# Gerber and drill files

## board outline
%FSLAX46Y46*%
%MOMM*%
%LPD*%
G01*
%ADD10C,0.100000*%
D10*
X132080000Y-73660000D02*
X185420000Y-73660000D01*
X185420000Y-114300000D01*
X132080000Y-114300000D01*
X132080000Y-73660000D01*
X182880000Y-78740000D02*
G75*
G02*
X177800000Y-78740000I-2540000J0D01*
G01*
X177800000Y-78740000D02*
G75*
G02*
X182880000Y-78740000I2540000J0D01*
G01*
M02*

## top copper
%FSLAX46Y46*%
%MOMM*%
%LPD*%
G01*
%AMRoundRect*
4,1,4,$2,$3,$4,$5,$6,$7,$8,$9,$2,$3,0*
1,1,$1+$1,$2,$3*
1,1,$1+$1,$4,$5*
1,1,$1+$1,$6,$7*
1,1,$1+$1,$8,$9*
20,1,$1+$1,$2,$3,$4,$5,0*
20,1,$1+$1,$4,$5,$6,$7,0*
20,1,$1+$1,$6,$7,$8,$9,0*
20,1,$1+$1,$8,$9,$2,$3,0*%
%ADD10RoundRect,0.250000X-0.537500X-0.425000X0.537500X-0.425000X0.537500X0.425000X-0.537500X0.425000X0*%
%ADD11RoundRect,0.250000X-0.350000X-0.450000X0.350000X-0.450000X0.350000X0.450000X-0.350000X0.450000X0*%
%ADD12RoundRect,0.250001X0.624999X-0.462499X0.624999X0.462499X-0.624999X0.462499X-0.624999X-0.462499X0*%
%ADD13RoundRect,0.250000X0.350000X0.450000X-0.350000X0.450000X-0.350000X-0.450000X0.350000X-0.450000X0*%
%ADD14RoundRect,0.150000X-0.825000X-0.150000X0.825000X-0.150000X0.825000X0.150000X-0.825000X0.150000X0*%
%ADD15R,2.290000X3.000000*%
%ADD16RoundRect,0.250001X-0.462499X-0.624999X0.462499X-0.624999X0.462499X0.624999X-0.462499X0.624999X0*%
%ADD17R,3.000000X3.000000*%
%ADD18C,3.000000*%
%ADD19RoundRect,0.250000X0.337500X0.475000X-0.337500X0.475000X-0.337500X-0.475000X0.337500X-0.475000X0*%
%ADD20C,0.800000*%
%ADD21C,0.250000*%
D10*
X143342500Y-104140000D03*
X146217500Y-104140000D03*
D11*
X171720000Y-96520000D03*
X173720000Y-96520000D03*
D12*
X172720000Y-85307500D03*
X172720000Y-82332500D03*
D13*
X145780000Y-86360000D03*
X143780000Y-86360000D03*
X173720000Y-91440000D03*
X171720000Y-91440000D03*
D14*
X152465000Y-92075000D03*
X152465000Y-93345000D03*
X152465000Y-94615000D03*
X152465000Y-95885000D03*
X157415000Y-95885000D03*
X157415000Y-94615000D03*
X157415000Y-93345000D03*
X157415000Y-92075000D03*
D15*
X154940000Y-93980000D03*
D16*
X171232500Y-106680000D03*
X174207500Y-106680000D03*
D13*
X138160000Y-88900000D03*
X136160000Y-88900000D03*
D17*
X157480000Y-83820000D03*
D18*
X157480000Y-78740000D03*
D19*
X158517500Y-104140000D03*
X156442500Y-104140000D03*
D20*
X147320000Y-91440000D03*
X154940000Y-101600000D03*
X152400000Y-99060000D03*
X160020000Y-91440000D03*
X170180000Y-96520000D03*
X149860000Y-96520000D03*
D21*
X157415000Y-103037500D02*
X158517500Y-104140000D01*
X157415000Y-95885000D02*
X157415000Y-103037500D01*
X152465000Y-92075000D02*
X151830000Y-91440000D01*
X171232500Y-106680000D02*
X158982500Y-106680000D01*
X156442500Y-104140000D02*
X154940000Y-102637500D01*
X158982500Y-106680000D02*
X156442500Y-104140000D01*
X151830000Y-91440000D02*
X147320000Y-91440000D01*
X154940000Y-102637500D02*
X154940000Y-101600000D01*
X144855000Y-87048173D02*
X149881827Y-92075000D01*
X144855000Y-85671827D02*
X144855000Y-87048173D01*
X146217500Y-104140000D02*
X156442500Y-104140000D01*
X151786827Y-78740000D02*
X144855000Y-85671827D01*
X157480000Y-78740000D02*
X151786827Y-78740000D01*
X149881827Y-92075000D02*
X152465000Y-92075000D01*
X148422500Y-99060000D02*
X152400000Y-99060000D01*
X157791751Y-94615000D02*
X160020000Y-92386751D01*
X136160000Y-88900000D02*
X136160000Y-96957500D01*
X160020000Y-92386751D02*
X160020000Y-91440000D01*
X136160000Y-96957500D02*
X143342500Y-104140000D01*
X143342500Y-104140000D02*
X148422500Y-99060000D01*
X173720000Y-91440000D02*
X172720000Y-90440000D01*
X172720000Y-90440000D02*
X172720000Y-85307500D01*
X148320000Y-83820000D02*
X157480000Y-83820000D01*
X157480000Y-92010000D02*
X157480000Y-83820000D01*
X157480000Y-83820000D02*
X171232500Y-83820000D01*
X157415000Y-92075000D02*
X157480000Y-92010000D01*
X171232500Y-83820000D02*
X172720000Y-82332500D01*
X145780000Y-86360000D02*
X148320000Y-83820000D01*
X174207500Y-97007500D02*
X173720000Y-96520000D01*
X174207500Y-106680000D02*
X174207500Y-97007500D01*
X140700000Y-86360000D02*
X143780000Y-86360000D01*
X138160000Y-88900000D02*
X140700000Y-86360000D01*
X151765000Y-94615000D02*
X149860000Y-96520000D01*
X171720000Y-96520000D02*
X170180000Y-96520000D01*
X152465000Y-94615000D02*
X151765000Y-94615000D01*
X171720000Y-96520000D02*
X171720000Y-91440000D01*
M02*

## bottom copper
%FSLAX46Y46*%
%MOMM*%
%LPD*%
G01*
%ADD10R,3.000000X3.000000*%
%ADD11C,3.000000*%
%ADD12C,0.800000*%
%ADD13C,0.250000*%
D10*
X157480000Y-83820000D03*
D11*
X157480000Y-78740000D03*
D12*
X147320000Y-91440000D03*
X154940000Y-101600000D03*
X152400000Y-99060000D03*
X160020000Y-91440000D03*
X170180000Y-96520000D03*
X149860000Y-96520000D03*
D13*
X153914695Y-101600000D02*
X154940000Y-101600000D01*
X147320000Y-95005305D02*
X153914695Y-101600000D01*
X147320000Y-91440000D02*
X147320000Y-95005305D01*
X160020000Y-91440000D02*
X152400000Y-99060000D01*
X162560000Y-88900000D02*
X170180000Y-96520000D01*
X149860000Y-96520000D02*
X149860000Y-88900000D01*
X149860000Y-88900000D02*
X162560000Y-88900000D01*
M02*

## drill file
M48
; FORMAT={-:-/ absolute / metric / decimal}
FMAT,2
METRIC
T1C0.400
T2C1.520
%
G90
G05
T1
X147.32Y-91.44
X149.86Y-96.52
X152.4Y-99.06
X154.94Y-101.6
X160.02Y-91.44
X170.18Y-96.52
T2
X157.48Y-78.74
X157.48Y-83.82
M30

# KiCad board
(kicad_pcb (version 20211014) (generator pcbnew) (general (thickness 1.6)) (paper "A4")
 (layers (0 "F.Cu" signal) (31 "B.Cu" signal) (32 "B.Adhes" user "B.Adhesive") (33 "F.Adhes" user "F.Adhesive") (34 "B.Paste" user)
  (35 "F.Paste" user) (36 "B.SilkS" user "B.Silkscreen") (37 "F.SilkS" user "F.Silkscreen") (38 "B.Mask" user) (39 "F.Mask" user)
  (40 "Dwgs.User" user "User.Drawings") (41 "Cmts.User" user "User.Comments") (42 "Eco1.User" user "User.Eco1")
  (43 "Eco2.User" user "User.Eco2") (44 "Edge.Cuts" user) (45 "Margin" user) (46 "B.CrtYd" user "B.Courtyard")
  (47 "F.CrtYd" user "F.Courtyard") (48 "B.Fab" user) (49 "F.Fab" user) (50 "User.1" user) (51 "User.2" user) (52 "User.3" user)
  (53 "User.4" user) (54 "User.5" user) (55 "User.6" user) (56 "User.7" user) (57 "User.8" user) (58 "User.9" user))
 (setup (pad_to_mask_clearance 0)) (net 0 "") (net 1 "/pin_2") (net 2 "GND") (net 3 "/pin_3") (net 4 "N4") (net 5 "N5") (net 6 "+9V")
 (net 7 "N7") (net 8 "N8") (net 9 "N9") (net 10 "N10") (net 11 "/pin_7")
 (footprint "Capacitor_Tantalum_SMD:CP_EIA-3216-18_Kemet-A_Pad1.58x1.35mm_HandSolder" (layer "F.Cu") (at 144.78 104.14)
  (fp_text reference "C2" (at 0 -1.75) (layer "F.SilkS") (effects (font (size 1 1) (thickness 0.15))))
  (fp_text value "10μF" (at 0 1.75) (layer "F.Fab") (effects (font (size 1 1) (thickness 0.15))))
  (pad "1" smd roundrect (at -1.4375 0) (size 1.575 1.35) (layers "F.Cu" "F.Paste" "F.Mask") (roundrect_rratio 0.185185) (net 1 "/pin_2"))
  (pad "2" smd roundrect (at 1.4375 0) (size 1.575 1.35) (layers "F.Cu" "F.Paste" "F.Mask") (roundrect_rratio 0.185185) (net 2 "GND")))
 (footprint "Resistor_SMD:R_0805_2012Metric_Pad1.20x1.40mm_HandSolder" (layer "F.Cu") (at 172.72 96.52)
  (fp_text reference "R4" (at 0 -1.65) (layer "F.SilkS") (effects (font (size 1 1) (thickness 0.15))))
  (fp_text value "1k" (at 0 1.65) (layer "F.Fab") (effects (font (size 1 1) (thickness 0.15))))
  (pad "1" smd roundrect (at -1 0) (size 1.2 1.4) (layers "F.Cu" "F.Paste" "F.Mask") (roundrect_rratio 0.208333) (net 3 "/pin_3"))
  (pad "2" smd roundrect (at 1 0) (size 1.2 1.4) (layers "F.Cu" "F.Paste" "F.Mask") (roundrect_rratio 0.208333) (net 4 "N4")))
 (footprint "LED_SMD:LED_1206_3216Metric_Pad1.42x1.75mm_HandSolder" (layer "F.Cu") (at 172.72 83.82 90)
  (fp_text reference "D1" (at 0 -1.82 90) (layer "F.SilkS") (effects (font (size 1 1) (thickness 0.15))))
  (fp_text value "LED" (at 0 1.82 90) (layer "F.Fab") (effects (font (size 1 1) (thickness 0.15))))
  (pad "1" smd roundrect (at -1.4875 0 90) (size 1.425 1.75) (layers "F.Cu" "F.Paste" "F.Mask") (roundrect_rratio 0.175439) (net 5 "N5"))
  (pad "2" smd roundrect (at 1.4875 0 90) (size 1.425 1.75) (layers "F.Cu" "F.Paste" "F.Mask") (roundrect_rratio 0.175439) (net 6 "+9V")))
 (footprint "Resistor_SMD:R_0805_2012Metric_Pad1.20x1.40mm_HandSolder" (layer "F.Cu") (at 144.78 86.36 180)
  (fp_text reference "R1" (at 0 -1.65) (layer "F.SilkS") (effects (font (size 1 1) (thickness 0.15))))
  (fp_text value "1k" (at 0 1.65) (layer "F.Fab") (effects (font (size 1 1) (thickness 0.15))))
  (pad "1" smd roundrect (at -1 0 180) (size 1.2 1.4) (layers "F.Cu" "F.Paste" "F.Mask") (roundrect_rratio 0.208333) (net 6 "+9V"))
  (pad "2" smd roundrect (at 1 0 180) (size 1.2 1.4) (layers "F.Cu" "F.Paste" "F.Mask") (roundrect_rratio 0.208333) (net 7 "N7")))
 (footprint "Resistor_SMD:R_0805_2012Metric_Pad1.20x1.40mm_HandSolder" (layer "F.Cu") (at 172.72 91.44 180)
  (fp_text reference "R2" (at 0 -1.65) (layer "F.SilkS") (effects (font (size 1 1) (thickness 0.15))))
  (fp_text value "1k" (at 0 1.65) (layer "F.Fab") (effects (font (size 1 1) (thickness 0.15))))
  (pad "1" smd roundrect (at -1 0 180) (size 1.2 1.4) (layers "F.Cu" "F.Paste" "F.Mask") (roundrect_rratio 0.208333) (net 5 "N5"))
  (pad "2" smd roundrect (at 1 0 180) (size 1.2 1.4) (layers "F.Cu" "F.Paste" "F.Mask") (roundrect_rratio 0.208333) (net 3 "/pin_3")))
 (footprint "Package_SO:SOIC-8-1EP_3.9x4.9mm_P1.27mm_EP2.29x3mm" (layer "F.Cu") (at 154.94 93.98)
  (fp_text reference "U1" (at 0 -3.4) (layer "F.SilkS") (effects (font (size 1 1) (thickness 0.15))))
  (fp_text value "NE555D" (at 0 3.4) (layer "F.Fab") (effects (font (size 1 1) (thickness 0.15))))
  (pad "" smd roundrect (at 0.57 -0.75) (size 0.92 1.21) (layers "F.Paste") (roundrect_rratio 0.25))
  (pad "" smd roundrect (at 0.57 0.75) (size 0.92 1.21) (layers "F.Paste") (roundrect_rratio 0.25))
  (pad "" smd roundrect (at -0.57 0.75) (size 0.92 1.21) (layers "F.Paste") (roundrect_rratio 0.25))
  (pad "" smd roundrect (at -0.57 -0.75) (size 0.92 1.21) (layers "F.Paste") (roundrect_rratio 0.25))
  (pad "1" smd roundrect (at -2.475 -1.905) (size 1.95 0.6) (layers "F.Cu" "F.Paste" "F.Mask") (roundrect_rratio 0.25) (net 2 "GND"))
  (pad "2" smd roundrect (at -2.475 -0.635) (size 1.95 0.6) (layers "F.Cu" "F.Paste" "F.Mask") (roundrect_rratio 0.25) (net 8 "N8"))
  (pad "3" smd roundrect (at -2.475 0.635) (size 1.95 0.6) (layers "F.Cu" "F.Paste" "F.Mask") (roundrect_rratio 0.25) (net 3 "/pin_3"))
  (pad "4" smd roundrect (at -2.475 1.905) (size 1.95 0.6) (layers "F.Cu" "F.Paste" "F.Mask") (roundrect_rratio 0.25) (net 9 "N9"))
  (pad "5" smd roundrect (at 2.475 1.905) (size 1.95 0.6) (layers "F.Cu" "F.Paste" "F.Mask") (roundrect_rratio 0.25) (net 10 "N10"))
  (pad "6" smd roundrect (at 2.475 0.635) (size 1.95 0.6) (layers "F.Cu" "F.Paste" "F.Mask") (roundrect_rratio 0.25) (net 1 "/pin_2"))
  (pad "7" smd roundrect (at 2.475 -0.635) (size 1.95 0.6) (layers "F.Cu" "F.Paste" "F.Mask") (roundrect_rratio 0.25) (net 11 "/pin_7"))
  (pad "8" smd roundrect (at 2.475 -1.905) (size 1.95 0.6) (layers "F.Cu" "F.Paste" "F.Mask") (roundrect_rratio 0.25) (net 6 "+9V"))
  (pad "9" smd rect (at 0 0) (size 2.29 3) (layers "F.Cu" "F.Mask")))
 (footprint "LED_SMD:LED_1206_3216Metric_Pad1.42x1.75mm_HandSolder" (layer "F.Cu") (at 172.72 106.68)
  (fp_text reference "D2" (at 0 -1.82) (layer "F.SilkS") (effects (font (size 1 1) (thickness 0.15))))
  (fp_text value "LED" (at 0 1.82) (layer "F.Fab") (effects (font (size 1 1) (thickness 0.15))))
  (pad "1" smd roundrect (at -1.4875 0) (size 1.425 1.75) (layers "F.Cu" "F.Paste" "F.Mask") (roundrect_rratio 0.175439) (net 2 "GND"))
  (pad "2" smd roundrect (at 1.4875 0) (size 1.425 1.75) (layers "F.Cu" "F.Paste" "F.Mask") (roundrect_rratio 0.175439) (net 4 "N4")))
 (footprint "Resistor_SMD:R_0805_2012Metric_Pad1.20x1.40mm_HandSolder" (layer "F.Cu") (at 137.16 88.9 180)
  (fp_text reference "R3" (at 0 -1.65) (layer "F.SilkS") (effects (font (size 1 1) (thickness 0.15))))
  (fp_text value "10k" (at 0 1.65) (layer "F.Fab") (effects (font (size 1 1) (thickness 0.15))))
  (pad "1" smd roundrect (at -1 0 180) (size 1.2 1.4) (layers "F.Cu" "F.Paste" "F.Mask") (roundrect_rratio 0.208333) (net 7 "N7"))
  (pad "2" smd roundrect (at 1 0 180) (size 1.2 1.4) (layers "F.Cu" "F.Paste" "F.Mask") (roundrect_rratio 0.208333) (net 1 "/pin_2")))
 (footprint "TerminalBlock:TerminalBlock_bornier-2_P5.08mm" (layer "F.Cu") (at 157.48 83.82 90)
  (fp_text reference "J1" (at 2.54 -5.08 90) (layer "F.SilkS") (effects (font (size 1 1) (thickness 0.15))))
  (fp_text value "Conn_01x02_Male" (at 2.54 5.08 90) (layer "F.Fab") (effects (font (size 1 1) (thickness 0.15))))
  (pad "1" thru_hole rect (at 0 0 90) (size 3 3) (drill 1.52) (layers *.Cu *.Mask) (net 6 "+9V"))
  (pad "2" thru_hole circle (at 5.08 0 90) (size 3 3) (drill 1.52) (layers *.Cu *.Mask) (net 2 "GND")))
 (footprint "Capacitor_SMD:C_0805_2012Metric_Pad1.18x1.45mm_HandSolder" (layer "F.Cu") (at 157.48 104.14 180)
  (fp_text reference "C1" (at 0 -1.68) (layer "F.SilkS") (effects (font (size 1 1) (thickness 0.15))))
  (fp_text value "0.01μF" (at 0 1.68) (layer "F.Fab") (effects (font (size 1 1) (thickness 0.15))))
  (pad "1" smd roundrect (at -1.0375 0 180) (size 1.175 1.45) (layers "F.Cu" "F.Paste" "F.Mask") (roundrect_rratio 0.212766) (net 10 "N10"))
  (pad "2" smd roundrect (at 1.0375 0 180) (size 1.175 1.45) (layers "F.Cu" "F.Paste" "F.Mask") (roundrect_rratio 0.212766) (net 2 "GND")))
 (gr_rect (start 185.42 114.3) (end 132.08 73.66) (layer "Edge.Cuts") (width 0.1) (fill none))
 (gr_circle (center 180.34 78.74) (end 180.34 81.28) (layer "Edge.Cuts") (width 0.1) (fill none))
 (segment (start 157.415 103.0375) (end 158.5175 104.14) (width 0.25) (layer "F.Cu") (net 10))
 (segment (start 157.415 95.885) (end 157.415 103.0375) (width 0.25) (layer "F.Cu") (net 10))
 (segment (start 152.465 92.075) (end 151.83 91.44) (width 0.25) (layer "F.Cu") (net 2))
 (segment (start 171.2325 106.68) (end 158.9825 106.68) (width 0.25) (layer "F.Cu") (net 2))
 (segment (start 156.4425 104.14) (end 154.94 102.6375) (width 0.25) (layer "F.Cu") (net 2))
 (segment (start 158.9825 106.68) (end 156.4425 104.14) (width 0.25) (layer "F.Cu") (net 2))
 (segment (start 151.83 91.44) (end 147.32 91.44) (width 0.25) (layer "F.Cu") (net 2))
 (segment (start 154.94 102.6375) (end 154.94 101.6) (width 0.25) (layer "F.Cu") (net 2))
 (segment (start 144.855 87.048173) (end 149.881827 92.075) (width 0.25) (layer "F.Cu") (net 2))
 (segment (start 144.855 85.671827) (end 144.855 87.048173) (width 0.25) (layer "F.Cu") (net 2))
 (segment (start 146.2175 104.14) (end 156.4425 104.14) (width 0.25) (layer "F.Cu") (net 2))
 (segment (start 151.786827 78.74) (end 144.855 85.671827) (width 0.25) (layer "F.Cu") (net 2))
 (segment (start 157.48 78.74) (end 151.786827 78.74) (width 0.25) (layer "F.Cu") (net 2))
 (segment (start 149.881827 92.075) (end 152.465 92.075) (width 0.25) (layer "F.Cu") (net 2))
 (via (at 147.32 91.44) (size 0.8) (drill 0.4) (layers "F.Cu" "B.Cu") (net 2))
 (via (at 154.94 101.6) (size 0.8) (drill 0.4) (layers "F.Cu" "B.Cu") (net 2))
 (segment (start 153.914695 101.6) (end 154.94 101.6) (width 0.25) (layer "B.Cu") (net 2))
 (segment (start 147.32 95.005305) (end 153.914695 101.6) (width 0.25) (layer "B.Cu") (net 2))
 (segment (start 147.32 91.44) (end 147.32 95.005305) (width 0.25) (layer "B.Cu") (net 2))
 (segment (start 148.4225 99.06) (end 152.4 99.06) (width 0.25) (layer "F.Cu") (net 1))
 (segment (start 157.791751 94.615) (end 160.02 92.386751) (width 0.25) (layer "F.Cu") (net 1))
 (segment (start 136.16 88.9) (end 136.16 96.9575) (width 0.25) (layer "F.Cu") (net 1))
 (segment (start 160.02 92.386751) (end 160.02 91.44) (width 0.25) (layer "F.Cu") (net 1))
 (segment (start 136.16 96.9575) (end 143.3425 104.14) (width 0.25) (layer "F.Cu") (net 1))
 (segment (start 143.3425 104.14) (end 148.4225 99.06) (width 0.25) (layer "F.Cu") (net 1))
 (via (at 152.4 99.06) (size 0.8) (drill 0.4) (layers "F.Cu" "B.Cu") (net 1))
 (via (at 160.02 91.44) (size 0.8) (drill 0.4) (layers "F.Cu" "B.Cu") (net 1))
 (segment (start 160.02 91.44) (end 152.4 99.06) (width 0.25) (layer "B.Cu") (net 1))
 (segment (start 173.72 91.44) (end 172.72 90.44) (width 0.25) (layer "F.Cu") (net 5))
 (segment (start 172.72 90.44) (end 172.72 85.3075) (width 0.25) (layer "F.Cu") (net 5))
 (segment (start 148.32 83.82) (end 157.48 83.82) (width 0.25) (layer "F.Cu") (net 6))
 (segment (start 157.48 92.01) (end 157.48 83.82) (width 0.25) (layer "F.Cu") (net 6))
 (segment (start 157.48 83.82) (end 171.2325 83.82) (width 0.25) (layer "F.Cu") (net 6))
 (segment (start 157.415 92.075) (end 157.48 92.01) (width 0.25) (layer "F.Cu") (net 6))
 (segment (start 171.2325 83.82) (end 172.72 82.3325) (width 0.25) (layer "F.Cu") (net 6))
 (segment (start 145.78 86.36) (end 148.32 83.82) (width 0.25) (layer "F.Cu") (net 6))
 (segment (start 174.2075 97.0075) (end 173.72 96.52) (width 0.25) (layer "F.Cu") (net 4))
 (segment (start 174.2075 106.68) (end 174.2075 97.0075) (width 0.25) (layer "F.Cu") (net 4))
 (segment (start 140.7 86.36) (end 143.78 86.36) (width 0.25) (layer "F.Cu") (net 7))
 (segment (start 138.16 88.9) (end 140.7 86.36) (width 0.25) (layer "F.Cu") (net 7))
 (segment (start 151.765 94.615) (end 149.86 96.52) (width 0.25) (layer "F.Cu") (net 3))
 (segment (start 171.72 96.52) (end 170.18 96.52) (width 0.25) (layer "F.Cu") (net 3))
 (segment (start 152.465 94.615) (end 151.765 94.615) (width 0.25) (layer "F.Cu") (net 3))
 (segment (start 171.72 96.52) (end 171.72 91.44) (width 0.25) (layer "F.Cu") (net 3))
 (via (at 170.18 96.52) (size 0.8) (drill 0.4) (layers "F.Cu" "B.Cu") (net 3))
 (via (at 149.86 96.52) (size 0.8) (drill 0.4) (layers "F.Cu" "B.Cu") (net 3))
 (segment (start 162.56 88.9) (end 170.18 96.52) (width 0.25) (layer "B.Cu") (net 3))
 (segment (start 149.86 96.52) (end 149.86 88.9) (width 0.25) (layer "B.Cu") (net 3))
 (segment (start 149.86 88.9) (end 162.56 88.9) (width 0.25) (layer "B.Cu") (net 3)))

